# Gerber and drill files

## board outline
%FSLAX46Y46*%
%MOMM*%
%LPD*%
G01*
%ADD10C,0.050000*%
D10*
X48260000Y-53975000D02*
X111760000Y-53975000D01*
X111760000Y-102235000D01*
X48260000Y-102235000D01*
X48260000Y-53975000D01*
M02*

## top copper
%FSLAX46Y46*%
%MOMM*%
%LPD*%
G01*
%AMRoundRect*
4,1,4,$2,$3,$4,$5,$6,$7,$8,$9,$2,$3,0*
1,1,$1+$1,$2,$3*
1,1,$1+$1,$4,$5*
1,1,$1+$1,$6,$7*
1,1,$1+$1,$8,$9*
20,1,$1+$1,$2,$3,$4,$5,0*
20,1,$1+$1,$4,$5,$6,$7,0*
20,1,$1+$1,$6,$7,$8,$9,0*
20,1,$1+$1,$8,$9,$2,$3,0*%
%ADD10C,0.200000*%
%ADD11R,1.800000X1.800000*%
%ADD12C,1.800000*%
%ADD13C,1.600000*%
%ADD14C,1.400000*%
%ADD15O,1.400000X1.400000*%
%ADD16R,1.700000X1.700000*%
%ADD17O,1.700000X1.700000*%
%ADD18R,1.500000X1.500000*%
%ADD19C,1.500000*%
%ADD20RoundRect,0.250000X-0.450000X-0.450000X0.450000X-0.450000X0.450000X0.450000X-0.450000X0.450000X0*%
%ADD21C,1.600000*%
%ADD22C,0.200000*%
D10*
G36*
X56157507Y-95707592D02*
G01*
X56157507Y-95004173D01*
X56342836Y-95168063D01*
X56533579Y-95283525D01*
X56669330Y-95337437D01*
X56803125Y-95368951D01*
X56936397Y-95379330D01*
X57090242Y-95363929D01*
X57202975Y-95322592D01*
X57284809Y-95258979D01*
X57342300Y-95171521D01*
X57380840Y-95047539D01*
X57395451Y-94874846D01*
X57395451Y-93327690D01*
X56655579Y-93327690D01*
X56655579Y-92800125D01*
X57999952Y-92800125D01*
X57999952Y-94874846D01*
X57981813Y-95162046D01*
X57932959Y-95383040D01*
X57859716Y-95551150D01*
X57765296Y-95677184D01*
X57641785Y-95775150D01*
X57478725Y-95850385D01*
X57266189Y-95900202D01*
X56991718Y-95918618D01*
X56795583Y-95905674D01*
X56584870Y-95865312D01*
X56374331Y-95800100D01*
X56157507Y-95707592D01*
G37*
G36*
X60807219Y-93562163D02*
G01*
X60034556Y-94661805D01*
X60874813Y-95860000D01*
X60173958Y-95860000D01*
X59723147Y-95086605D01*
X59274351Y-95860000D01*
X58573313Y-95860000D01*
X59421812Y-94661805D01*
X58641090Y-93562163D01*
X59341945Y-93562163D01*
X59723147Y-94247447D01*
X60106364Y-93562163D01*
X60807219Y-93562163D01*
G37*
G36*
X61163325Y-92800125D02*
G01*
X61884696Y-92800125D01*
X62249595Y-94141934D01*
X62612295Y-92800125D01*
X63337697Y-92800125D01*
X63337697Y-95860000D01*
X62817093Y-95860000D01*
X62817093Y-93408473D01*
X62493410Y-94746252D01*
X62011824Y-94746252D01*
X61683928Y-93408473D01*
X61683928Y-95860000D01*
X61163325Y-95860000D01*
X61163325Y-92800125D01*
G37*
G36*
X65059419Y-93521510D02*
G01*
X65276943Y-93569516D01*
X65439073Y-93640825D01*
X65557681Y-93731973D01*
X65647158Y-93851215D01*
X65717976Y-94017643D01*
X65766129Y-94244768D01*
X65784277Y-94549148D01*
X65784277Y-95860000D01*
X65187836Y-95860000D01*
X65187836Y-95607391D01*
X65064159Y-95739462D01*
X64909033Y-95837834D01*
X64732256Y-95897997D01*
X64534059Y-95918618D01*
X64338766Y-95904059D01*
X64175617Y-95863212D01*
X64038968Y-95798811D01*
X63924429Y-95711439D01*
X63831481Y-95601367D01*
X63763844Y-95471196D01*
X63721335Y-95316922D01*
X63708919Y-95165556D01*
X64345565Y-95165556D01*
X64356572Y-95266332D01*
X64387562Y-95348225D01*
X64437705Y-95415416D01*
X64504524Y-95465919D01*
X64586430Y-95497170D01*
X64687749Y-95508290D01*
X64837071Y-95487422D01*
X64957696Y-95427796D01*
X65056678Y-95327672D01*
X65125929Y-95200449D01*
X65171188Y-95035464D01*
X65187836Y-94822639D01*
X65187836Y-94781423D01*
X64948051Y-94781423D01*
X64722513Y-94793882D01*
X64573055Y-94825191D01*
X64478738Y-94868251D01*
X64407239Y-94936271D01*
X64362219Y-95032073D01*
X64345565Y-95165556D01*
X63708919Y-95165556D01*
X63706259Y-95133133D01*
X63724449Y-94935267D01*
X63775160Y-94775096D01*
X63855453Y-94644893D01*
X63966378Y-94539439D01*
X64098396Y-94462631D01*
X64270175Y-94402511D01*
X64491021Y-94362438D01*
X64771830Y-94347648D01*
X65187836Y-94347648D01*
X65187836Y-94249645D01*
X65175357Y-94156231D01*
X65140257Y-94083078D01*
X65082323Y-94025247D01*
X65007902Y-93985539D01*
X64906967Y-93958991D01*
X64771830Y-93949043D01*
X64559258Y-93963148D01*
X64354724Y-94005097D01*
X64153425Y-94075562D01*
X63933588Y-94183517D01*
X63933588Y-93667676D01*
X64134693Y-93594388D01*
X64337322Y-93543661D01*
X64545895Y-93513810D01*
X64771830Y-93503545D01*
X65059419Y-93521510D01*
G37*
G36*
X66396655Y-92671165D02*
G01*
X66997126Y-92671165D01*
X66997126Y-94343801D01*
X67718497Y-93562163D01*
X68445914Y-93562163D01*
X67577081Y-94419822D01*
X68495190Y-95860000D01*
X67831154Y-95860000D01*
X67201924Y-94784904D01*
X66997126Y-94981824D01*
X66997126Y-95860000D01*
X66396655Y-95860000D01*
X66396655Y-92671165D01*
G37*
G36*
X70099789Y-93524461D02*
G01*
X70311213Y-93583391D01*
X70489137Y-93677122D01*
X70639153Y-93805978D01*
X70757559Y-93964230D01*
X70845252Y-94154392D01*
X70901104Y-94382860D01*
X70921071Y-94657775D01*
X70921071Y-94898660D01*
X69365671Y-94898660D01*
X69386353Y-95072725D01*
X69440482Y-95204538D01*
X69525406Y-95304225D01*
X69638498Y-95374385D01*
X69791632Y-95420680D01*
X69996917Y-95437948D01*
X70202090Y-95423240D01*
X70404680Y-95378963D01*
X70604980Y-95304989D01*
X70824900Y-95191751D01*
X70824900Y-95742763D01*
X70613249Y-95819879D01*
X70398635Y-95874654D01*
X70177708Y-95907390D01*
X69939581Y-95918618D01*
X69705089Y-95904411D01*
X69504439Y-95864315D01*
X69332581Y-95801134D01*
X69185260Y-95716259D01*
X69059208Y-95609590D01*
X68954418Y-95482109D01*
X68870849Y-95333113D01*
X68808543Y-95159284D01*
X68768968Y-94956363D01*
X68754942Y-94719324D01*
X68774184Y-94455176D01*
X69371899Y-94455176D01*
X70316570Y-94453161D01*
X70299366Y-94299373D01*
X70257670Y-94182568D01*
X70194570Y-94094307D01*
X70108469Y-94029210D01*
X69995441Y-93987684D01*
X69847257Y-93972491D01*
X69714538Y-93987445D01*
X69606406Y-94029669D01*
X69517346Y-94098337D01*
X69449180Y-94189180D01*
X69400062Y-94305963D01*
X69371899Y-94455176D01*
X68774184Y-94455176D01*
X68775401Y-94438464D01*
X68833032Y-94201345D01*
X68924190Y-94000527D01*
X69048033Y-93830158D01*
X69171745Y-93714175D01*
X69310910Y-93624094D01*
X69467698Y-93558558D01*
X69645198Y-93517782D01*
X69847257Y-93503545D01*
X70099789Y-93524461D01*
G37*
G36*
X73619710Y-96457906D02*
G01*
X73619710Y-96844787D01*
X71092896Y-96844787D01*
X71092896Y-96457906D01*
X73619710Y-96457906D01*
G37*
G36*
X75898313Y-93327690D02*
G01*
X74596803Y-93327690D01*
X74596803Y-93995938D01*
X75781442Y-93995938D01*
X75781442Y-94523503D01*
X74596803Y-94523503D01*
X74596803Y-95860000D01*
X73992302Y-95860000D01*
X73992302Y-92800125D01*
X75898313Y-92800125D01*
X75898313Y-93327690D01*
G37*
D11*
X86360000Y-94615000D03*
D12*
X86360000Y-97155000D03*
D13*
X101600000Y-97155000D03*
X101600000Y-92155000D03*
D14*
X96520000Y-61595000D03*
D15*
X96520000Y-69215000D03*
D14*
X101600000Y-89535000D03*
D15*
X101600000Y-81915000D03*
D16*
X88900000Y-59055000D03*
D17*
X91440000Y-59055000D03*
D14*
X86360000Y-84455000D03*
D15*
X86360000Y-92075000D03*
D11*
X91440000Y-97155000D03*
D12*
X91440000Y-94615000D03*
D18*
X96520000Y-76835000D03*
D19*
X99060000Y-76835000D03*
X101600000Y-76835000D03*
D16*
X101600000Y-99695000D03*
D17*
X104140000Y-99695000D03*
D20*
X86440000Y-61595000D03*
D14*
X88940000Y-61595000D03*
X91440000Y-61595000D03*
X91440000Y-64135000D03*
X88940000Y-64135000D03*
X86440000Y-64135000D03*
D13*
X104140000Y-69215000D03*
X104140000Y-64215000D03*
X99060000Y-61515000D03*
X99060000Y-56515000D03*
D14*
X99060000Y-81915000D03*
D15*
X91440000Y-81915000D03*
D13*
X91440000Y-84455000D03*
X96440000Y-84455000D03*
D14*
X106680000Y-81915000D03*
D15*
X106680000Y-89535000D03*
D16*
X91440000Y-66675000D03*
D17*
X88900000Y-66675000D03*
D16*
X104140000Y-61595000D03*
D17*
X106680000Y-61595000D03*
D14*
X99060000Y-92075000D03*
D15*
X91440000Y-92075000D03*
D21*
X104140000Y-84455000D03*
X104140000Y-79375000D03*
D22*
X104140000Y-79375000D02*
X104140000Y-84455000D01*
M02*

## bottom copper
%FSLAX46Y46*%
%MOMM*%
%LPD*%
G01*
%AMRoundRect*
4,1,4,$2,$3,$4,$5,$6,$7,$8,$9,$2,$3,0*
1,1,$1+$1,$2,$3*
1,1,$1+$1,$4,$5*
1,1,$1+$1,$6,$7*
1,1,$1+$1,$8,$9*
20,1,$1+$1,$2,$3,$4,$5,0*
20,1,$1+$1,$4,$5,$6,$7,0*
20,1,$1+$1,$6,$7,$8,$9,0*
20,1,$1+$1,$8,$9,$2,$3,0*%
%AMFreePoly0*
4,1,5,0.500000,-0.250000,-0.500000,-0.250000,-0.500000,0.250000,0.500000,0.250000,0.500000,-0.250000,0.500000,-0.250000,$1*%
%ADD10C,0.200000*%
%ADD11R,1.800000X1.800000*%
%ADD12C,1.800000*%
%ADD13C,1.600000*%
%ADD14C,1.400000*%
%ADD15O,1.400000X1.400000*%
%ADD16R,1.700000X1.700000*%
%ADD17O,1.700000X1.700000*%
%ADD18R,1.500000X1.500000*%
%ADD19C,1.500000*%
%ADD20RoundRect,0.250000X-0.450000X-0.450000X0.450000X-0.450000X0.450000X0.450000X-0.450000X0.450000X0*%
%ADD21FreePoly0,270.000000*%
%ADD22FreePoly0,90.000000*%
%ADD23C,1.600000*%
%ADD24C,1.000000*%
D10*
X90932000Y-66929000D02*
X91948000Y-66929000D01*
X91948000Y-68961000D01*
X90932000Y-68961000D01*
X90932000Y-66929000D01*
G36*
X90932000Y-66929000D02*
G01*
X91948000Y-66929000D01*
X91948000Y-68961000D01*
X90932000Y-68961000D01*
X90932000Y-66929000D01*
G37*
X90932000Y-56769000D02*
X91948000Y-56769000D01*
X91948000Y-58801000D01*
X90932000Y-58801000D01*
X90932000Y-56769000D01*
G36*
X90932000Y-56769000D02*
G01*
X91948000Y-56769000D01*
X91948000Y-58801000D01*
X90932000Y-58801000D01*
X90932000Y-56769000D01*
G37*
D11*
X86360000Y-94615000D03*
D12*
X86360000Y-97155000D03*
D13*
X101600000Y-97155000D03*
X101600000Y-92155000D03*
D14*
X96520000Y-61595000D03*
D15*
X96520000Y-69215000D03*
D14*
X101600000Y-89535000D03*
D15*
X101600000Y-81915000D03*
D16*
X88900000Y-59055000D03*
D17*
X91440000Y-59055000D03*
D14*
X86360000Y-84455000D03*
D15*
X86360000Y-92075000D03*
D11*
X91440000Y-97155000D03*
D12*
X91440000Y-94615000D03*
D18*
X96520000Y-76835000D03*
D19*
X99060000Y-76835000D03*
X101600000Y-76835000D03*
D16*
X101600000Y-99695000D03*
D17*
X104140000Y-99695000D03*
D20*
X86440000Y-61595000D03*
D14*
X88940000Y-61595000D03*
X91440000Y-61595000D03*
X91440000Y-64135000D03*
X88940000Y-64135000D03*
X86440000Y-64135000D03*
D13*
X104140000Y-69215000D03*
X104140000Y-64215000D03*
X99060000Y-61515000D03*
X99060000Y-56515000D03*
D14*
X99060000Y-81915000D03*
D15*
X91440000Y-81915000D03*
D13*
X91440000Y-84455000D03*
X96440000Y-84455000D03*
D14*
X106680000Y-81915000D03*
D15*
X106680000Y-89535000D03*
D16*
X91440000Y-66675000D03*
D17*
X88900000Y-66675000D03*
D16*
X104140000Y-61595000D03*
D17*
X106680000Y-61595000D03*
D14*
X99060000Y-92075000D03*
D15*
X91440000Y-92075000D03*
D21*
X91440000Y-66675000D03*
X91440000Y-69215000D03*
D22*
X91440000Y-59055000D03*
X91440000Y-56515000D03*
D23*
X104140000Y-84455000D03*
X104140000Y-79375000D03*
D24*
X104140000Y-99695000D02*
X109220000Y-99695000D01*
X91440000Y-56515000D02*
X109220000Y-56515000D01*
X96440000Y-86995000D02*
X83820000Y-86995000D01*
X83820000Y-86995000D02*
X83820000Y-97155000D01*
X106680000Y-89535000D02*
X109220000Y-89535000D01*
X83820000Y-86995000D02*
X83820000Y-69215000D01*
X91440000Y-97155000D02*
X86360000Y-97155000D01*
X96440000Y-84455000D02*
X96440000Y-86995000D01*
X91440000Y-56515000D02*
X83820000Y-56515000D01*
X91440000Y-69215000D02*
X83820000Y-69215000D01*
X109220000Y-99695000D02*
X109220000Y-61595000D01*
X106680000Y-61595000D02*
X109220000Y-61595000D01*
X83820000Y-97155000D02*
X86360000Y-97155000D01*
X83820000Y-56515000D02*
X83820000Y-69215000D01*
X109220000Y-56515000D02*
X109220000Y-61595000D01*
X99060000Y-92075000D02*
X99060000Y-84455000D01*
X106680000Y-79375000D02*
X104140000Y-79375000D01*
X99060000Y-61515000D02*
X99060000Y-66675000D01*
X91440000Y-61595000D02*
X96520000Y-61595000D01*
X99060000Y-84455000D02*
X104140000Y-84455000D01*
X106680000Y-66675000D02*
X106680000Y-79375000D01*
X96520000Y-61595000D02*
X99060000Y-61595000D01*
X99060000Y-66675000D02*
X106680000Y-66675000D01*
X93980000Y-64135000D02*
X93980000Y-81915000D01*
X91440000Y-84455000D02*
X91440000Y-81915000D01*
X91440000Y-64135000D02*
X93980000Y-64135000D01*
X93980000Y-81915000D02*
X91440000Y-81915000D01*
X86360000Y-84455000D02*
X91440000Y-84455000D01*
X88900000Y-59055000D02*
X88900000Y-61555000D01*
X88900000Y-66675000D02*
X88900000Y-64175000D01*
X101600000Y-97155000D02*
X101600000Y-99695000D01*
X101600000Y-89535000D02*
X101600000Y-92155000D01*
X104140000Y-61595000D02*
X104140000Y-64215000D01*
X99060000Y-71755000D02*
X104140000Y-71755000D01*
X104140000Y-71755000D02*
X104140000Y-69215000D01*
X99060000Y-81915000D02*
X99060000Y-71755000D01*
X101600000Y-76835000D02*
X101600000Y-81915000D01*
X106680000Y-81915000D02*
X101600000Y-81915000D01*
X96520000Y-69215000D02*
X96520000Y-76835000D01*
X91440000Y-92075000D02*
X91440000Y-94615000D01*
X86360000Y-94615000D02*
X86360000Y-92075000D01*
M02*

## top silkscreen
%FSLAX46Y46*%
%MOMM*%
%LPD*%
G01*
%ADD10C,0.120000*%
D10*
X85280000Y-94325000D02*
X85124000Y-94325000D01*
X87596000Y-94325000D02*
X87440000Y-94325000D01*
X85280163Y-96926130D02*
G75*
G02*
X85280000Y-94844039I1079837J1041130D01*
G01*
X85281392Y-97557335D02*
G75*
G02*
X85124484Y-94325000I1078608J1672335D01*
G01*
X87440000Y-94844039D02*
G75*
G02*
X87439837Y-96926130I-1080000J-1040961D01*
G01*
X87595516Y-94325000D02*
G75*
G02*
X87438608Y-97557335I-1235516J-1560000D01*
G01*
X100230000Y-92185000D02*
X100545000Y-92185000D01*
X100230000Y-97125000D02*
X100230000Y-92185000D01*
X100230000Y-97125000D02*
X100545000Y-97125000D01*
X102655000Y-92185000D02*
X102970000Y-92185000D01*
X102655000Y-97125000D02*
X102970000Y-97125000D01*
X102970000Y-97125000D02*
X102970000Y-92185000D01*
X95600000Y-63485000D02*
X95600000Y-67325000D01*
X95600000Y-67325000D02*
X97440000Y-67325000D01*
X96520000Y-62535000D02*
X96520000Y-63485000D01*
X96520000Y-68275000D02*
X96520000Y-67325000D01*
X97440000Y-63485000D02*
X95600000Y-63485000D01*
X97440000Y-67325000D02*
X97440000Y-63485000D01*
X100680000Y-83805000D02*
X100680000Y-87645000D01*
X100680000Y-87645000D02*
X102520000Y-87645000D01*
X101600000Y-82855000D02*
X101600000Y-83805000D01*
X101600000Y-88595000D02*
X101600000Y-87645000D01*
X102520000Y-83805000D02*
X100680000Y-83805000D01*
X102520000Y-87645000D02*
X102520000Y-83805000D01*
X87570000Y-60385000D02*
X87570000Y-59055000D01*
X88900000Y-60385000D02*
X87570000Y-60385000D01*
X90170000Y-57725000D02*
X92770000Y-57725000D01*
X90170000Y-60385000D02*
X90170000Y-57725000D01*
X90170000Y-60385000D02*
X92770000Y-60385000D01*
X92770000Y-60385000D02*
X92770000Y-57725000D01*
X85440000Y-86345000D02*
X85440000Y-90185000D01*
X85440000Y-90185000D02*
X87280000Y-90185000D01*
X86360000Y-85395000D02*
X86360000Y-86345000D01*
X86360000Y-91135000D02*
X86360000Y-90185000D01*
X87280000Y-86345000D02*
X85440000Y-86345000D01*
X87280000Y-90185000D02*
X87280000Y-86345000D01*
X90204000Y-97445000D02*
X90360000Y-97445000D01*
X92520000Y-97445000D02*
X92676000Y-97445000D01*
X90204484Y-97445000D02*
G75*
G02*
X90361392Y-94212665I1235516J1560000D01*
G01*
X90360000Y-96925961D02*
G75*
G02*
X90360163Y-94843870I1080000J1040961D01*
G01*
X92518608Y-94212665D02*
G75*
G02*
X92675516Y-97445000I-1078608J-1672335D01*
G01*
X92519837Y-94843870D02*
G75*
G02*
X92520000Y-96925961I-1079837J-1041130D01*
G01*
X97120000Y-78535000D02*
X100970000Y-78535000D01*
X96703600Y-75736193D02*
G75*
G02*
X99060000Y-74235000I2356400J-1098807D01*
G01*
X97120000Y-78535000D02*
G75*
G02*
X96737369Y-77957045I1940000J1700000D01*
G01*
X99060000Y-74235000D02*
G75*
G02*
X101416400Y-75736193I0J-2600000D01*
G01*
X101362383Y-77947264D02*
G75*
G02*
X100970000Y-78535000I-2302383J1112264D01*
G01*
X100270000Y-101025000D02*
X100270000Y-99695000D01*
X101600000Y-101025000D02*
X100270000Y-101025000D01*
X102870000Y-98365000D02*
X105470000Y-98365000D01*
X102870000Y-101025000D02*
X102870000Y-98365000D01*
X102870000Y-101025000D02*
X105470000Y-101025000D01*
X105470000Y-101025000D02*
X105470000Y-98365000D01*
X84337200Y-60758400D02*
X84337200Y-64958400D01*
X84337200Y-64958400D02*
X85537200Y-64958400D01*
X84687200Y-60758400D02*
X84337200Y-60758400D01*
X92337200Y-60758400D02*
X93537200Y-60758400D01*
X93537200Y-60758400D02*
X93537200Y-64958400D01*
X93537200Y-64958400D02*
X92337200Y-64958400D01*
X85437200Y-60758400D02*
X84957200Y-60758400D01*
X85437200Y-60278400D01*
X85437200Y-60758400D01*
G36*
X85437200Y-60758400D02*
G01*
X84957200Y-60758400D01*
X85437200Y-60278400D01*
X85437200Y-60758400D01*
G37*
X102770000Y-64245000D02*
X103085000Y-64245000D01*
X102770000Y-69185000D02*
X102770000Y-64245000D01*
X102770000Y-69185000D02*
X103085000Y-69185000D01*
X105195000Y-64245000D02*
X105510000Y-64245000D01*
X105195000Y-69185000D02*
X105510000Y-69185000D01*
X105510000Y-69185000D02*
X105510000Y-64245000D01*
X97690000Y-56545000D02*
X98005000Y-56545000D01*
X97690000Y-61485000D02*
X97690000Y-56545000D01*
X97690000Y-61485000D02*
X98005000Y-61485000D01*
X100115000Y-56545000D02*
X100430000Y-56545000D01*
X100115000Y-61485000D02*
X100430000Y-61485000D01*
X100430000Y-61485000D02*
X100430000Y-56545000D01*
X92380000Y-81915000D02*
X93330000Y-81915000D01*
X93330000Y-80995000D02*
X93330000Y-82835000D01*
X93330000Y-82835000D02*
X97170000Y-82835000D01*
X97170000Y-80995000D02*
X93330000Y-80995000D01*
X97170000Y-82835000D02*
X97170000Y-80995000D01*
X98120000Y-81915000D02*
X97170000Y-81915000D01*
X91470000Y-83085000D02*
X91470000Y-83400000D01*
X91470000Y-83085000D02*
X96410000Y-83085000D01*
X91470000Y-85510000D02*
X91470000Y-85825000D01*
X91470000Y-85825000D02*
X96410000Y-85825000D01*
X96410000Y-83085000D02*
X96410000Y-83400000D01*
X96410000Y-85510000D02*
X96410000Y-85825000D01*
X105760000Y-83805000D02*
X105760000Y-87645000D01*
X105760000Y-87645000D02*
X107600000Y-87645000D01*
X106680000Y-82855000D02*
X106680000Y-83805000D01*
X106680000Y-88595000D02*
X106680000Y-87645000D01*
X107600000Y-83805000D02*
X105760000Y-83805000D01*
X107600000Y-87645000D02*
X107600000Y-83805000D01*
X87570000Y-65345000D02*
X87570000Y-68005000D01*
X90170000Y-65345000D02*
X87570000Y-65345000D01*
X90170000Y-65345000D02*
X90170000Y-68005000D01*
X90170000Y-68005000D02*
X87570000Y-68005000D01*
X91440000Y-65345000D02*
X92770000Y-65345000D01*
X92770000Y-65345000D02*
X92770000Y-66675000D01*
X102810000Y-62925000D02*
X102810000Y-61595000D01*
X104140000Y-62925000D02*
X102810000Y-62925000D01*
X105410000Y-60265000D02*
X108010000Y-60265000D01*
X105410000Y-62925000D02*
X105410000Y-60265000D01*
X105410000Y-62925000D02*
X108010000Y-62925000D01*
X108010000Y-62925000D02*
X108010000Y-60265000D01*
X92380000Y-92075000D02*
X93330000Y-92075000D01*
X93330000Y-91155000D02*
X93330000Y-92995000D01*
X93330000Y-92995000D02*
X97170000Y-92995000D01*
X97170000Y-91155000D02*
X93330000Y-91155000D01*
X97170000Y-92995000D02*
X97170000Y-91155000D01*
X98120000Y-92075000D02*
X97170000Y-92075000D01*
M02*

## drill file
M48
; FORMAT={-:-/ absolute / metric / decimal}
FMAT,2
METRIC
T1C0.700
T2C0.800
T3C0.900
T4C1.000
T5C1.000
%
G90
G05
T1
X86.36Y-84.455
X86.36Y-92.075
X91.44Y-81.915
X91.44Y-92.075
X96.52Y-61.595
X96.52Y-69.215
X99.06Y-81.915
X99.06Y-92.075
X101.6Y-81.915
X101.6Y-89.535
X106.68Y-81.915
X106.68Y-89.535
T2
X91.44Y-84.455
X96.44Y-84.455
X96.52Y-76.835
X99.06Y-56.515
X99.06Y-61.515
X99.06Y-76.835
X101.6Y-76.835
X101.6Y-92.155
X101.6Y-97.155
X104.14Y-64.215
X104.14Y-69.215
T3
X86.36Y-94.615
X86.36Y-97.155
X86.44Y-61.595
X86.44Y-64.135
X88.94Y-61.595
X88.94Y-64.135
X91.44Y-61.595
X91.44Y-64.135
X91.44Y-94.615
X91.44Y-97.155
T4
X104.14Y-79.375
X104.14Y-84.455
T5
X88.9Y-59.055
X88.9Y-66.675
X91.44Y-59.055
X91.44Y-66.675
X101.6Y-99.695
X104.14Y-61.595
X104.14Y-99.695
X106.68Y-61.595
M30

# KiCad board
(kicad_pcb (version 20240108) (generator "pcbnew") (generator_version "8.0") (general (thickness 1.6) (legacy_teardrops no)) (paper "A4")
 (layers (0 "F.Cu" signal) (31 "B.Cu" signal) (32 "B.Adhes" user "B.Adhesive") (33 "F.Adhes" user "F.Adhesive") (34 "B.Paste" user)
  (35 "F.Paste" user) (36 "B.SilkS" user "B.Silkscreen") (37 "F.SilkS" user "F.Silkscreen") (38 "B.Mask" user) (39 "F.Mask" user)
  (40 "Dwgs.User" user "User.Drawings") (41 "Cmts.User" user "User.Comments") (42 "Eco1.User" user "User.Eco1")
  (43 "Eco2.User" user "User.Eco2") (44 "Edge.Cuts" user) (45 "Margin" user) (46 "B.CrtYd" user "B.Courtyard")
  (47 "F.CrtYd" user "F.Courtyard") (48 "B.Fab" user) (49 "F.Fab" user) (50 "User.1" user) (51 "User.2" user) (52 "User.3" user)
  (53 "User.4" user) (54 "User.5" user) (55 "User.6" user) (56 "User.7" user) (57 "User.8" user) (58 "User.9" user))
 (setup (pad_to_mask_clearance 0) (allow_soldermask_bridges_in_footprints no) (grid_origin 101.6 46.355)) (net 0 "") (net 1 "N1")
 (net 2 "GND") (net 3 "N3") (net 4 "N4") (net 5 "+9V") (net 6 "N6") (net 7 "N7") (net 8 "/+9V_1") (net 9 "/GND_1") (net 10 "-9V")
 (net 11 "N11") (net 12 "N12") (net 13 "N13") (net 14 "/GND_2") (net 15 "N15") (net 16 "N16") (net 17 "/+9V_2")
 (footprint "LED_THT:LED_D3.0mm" (layer "F.Cu") (at 86.36 94.615 -90)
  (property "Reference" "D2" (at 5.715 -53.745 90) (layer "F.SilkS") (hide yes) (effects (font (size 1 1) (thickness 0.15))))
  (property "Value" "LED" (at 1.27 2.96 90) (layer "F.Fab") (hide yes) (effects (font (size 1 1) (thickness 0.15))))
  (fp_line (start -0.29 1.08) (end -0.29 1.236) (stroke (width 0.12) (type solid)) (layer "F.SilkS"))
  (fp_line (start -0.29 -1.236) (end -0.29 -1.08) (stroke (width 0.12) (type solid)) (layer "F.SilkS"))
  (fp_arc (start 2.31113 1.079837) (mid 1.270117 1.5) (end 0.229039 1.08) (stroke (width 0.12) (type solid)) (layer "F.SilkS"))
  (fp_arc (start 2.942335 1.078608) (mid 1.366487 1.987659) (end -0.29 1.235516) (stroke (width 0.12) (type solid)) (layer "F.SilkS"))
  (fp_arc (start 0.229039 -1.08) (mid 1.270117 -1.5) (end 2.31113 -1.079837) (stroke (width 0.12) (type solid)) (layer "F.SilkS"))
  (fp_arc (start -0.29 -1.235516) (mid 1.366487 -1.987659) (end 2.942335 -1.078608) (stroke (width 0.12) (type solid)) (layer "F.SilkS"))
  (pad "1" thru_hole rect (at 0 0 270) (size 1.8 1.8) (drill 0.9) (layers "*.Cu" "*.Mask") (remove_unused_layers no) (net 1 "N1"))
  (pad "2" thru_hole circle (at 2.54 0 270) (size 1.8 1.8) (drill 0.9) (layers "*.Cu" "*.Mask") (remove_unused_layers no) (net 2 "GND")))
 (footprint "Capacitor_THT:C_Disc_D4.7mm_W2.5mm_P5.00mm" (layer "F.Cu") (at 101.6 97.155 90)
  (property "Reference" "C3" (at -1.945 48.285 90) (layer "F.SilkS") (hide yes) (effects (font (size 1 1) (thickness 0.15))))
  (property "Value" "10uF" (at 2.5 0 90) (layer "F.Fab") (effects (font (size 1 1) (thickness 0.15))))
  (fp_line (start 4.97 -1.37) (end 4.97 -1.055) (stroke (width 0.12) (type solid)) (layer "F.SilkS"))
  (fp_line (start 0.03 -1.37) (end 4.97 -1.37) (stroke (width 0.12) (type solid)) (layer "F.SilkS"))
  (fp_line (start 0.03 -1.37) (end 0.03 -1.055) (stroke (width 0.12) (type solid)) (layer "F.SilkS"))
  (fp_line (start 4.97 1.055) (end 4.97 1.37) (stroke (width 0.12) (type solid)) (layer "F.SilkS"))
  (fp_line (start 0.03 1.055) (end 0.03 1.37) (stroke (width 0.12) (type solid)) (layer "F.SilkS"))
  (fp_line (start 0.03 1.37) (end 4.97 1.37) (stroke (width 0.12) (type solid)) (layer "F.SilkS"))
  (pad "1" thru_hole circle (at 0 0 90) (size 1.6 1.6) (drill 0.8) (layers "*.Cu" "*.Mask") (remove_unused_layers no) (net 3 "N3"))
  (pad "2" thru_hole circle (at 5 0 90) (size 1.6 1.6) (drill 0.8) (layers "*.Cu" "*.Mask") (remove_unused_layers no) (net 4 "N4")))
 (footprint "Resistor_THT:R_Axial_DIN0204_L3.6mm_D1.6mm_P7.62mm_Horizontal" (layer "F.Cu") (at 96.52 61.595 -90)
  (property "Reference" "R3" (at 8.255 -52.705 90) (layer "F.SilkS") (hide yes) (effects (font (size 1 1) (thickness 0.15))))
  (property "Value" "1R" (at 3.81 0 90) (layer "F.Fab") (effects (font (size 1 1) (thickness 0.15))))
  (fp_line (start 1.89 0.92) (end 5.73 0.92) (stroke (width 0.12) (type solid)) (layer "F.SilkS"))
  (fp_line (start 5.73 0.92) (end 5.73 -0.92) (stroke (width 0.12) (type solid)) (layer "F.SilkS"))
  (fp_line (start 0.94 0) (end 1.89 0) (stroke (width 0.12) (type solid)) (layer "F.SilkS"))
  (fp_line (start 6.68 0) (end 5.73 0) (stroke (width 0.12) (type solid)) (layer "F.SilkS"))
  (fp_line (start 1.89 -0.92) (end 1.89 0.92) (stroke (width 0.12) (type solid)) (layer "F.SilkS"))
  (fp_line (start 5.73 -0.92) (end 1.89 -0.92) (stroke (width 0.12) (type solid)) (layer "F.SilkS"))
  (pad "1" thru_hole circle (at 0 0 270) (size 1.4 1.4) (drill 0.7) (layers "*.Cu" "*.Mask") (remove_unused_layers no) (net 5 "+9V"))
  (pad "2" thru_hole oval (at 7.62 0 270) (size 1.4 1.4) (drill 0.7) (layers "*.Cu" "*.Mask") (remove_unused_layers no) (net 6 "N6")))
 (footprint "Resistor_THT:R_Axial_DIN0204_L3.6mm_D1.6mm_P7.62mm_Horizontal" (layer "F.Cu") (at 101.6 89.535 90)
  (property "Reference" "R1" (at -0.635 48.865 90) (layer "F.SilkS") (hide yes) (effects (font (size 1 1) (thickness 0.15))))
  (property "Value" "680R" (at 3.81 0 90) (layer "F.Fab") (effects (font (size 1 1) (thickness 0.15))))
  (fp_line (start 5.73 -0.92) (end 1.89 -0.92) (stroke (width 0.12) (type solid)) (layer "F.SilkS"))
  (fp_line (start 1.89 -0.92) (end 1.89 0.92) (stroke (width 0.12) (type solid)) (layer "F.SilkS"))
  (fp_line (start 6.68 0) (end 5.73 0) (stroke (width 0.12) (type solid)) (layer "F.SilkS"))
  (fp_line (start 0.94 0) (end 1.89 0) (stroke (width 0.12) (type solid)) (layer "F.SilkS"))
  (fp_line (start 5.73 0.92) (end 5.73 -0.92) (stroke (width 0.12) (type solid)) (layer "F.SilkS"))
  (fp_line (start 1.89 0.92) (end 5.73 0.92) (stroke (width 0.12) (type solid)) (layer "F.SilkS"))
  (pad "1" thru_hole circle (at 0 0 90) (size 1.4 1.4) (drill 0.7) (layers "*.Cu" "*.Mask") (remove_unused_layers no) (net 4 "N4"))
  (pad "2" thru_hole oval (at 7.62 0 90) (size 1.4 1.4) (drill 0.7) (layers "*.Cu" "*.Mask") (remove_unused_layers no) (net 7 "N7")))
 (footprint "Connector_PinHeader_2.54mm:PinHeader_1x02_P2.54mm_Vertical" (layer "F.Cu") (at 88.9 59.055 90)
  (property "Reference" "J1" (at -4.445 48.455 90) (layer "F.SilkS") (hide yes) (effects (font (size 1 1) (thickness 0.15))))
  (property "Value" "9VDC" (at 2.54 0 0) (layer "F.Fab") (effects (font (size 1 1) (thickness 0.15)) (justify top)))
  (fp_line (start -1.33 -1.33) (end 0 -1.33) (stroke (width 0.12) (type solid)) (layer "F.SilkS"))
  (fp_line (start -1.33 0) (end -1.33 -1.33) (stroke (width 0.12) (type solid)) (layer "F.SilkS"))
  (fp_line (start 1.33 1.27) (end 1.33 3.87) (stroke (width 0.12) (type solid)) (layer "F.SilkS"))
  (fp_line (start -1.33 1.27) (end 1.33 1.27) (stroke (width 0.12) (type solid)) (layer "F.SilkS"))
  (fp_line (start -1.33 1.27) (end -1.33 3.87) (stroke (width 0.12) (type solid)) (layer "F.SilkS"))
  (fp_line (start -1.33 3.87) (end 1.33 3.87) (stroke (width 0.12) (type solid)) (layer "F.SilkS"))
  (pad "1" thru_hole rect (at 0 0 90) (size 1.7 1.7) (drill 1) (layers "*.Cu" "*.Mask") (remove_unused_layers no) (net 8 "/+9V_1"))
  (pad "2" thru_hole oval (at 0 2.54 90) (size 1.7 1.7) (drill 1) (layers "*.Cu" "*.Mask") (remove_unused_layers no) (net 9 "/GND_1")))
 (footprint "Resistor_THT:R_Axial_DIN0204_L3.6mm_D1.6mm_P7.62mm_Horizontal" (layer "F.Cu") (at 86.36 84.455 -90)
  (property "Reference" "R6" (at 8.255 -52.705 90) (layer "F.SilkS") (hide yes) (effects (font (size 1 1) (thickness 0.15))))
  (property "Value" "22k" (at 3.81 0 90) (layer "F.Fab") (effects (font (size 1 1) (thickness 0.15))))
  (fp_line (start 1.89 0.92) (end 5.73 0.92) (stroke (width 0.12) (type solid)) (layer "F.SilkS"))
  (fp_line (start 5.73 0.92) (end 5.73 -0.92) (stroke (width 0.12) (type solid)) (layer "F.SilkS"))
  (fp_line (start 0.94 0) (end 1.89 0) (stroke (width 0.12) (type solid)) (layer "F.SilkS"))
  (fp_line (start 6.68 0) (end 5.73 0) (stroke (width 0.12) (type solid)) (layer "F.SilkS"))
  (fp_line (start 1.89 -0.92) (end 1.89 0.92) (stroke (width 0.12) (type solid)) (layer "F.SilkS"))
  (fp_line (start 5.73 -0.92) (end 1.89 -0.92) (stroke (width 0.12) (type solid)) (layer "F.SilkS"))
  (pad "1" thru_hole circle (at 0 0 270) (size 1.4 1.4) (drill 0.7) (layers "*.Cu" "*.Mask") (remove_unused_layers no) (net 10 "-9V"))
  (pad "2" thru_hole oval (at 7.62 0 270) (size 1.4 1.4) (drill 0.7) (layers "*.Cu" "*.Mask") (remove_unused_layers no) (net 1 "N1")))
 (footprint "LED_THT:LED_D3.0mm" (layer "F.Cu") (at 91.44 97.155 90)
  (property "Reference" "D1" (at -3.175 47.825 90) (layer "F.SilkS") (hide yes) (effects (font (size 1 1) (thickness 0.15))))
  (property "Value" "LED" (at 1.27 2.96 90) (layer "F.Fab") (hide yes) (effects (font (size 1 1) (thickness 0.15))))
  (fp_line (start -0.29 -1.236) (end -0.29 -1.08) (stroke (width 0.12) (type solid)) (layer "F.SilkS"))
  (fp_line (start -0.29 1.08) (end -0.29 1.236) (stroke (width 0.12) (type solid)) (layer "F.SilkS"))
  (fp_arc (start -0.29 -1.235516) (mid 1.366487 -1.987659) (end 2.942335 -1.078608) (stroke (width 0.12) (type solid)) (layer "F.SilkS"))
  (fp_arc (start 0.229039 -1.08) (mid 1.270117 -1.5) (end 2.31113 -1.079837) (stroke (width 0.12) (type solid)) (layer "F.SilkS"))
  (fp_arc (start 2.942335 1.078608) (mid 1.366487 1.987659) (end -0.29 1.235516) (stroke (width 0.12) (type solid)) (layer "F.SilkS"))
  (fp_arc (start 2.31113 1.079837) (mid 1.270117 1.5) (end 0.229039 1.08) (stroke (width 0.12) (type solid)) (layer "F.SilkS"))
  (pad "1" thru_hole rect (at 0 0 90) (size 1.8 1.8) (drill 0.9) (layers "*.Cu" "*.Mask") (remove_unused_layers no) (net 2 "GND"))
  (pad "2" thru_hole circle (at 2.54 0 90) (size 1.8 1.8) (drill 0.9) (layers "*.Cu" "*.Mask") (remove_unused_layers no) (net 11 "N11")))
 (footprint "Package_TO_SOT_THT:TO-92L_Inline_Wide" (layer "F.Cu") (at 96.52 76.835)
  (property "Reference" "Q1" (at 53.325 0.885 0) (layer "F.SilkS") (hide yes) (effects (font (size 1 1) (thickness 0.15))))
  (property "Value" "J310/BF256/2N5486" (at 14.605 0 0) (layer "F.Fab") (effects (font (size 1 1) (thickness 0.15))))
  (fp_line (start 0.6 1.7) (end 4.45 1.7) (stroke (width 0.12) (type solid)) (layer "F.SilkS"))
  (fp_arc (start 0.1836 -1.098807) (mid 1.143021 -2.192817) (end 2.54 -2.6) (stroke (width 0.12) (type solid)) (layer "F.SilkS"))
  (fp_arc (start 0.6 1.7) (mid 0.389183 1.423933) (end 0.217369 1.122045) (stroke (width 0.12) (type solid)) (layer "F.SilkS"))
  (fp_arc (start 2.54 -2.6) (mid 3.936979 -2.192818) (end 4.8964 -1.098807) (stroke (width 0.12) (type solid)) (layer "F.SilkS"))
  (fp_arc (start 4.842383 1.112264) (mid 4.666594 1.419753) (end 4.45 1.7) (stroke (width 0.12) (type solid)) (layer "F.SilkS"))
  (pad "1" thru_hole rect (at 0 0) (size 1.5 1.5) (drill 0.8) (layers "*.Cu" "*.Mask") (remove_unused_layers no) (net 6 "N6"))
  (pad "2" thru_hole circle (at 2.54 0) (size 1.5 1.5) (drill 0.8) (layers "*.Cu" "*.Mask") (remove_unused_layers no) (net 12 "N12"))
  (pad "3" thru_hole circle (at 5.08 0) (size 1.5 1.5) (drill 0.8) (layers "*.Cu" "*.Mask") (remove_unused_layers no) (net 7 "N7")))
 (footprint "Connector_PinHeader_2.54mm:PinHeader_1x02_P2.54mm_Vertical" (layer "F.Cu") (at 101.6 99.695 90)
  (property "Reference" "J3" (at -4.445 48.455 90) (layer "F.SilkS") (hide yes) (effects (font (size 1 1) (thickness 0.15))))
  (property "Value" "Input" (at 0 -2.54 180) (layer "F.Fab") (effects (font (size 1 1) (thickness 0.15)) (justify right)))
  (fp_line (start -1.33 -1.33) (end 0 -1.33) (stroke (width 0.12) (type solid)) (layer "F.SilkS"))
  (fp_line (start -1.33 0) (end -1.33 -1.33) (stroke (width 0.12) (type solid)) (layer "F.SilkS"))
  (fp_line (start 1.33 1.27) (end 1.33 3.87) (stroke (width 0.12) (type solid)) (layer "F.SilkS"))
  (fp_line (start -1.33 1.27) (end 1.33 1.27) (stroke (width 0.12) (type solid)) (layer "F.SilkS"))
  (fp_line (start -1.33 1.27) (end -1.33 3.87) (stroke (width 0.12) (type solid)) (layer "F.SilkS"))
  (fp_line (start -1.33 3.87) (end 1.33 3.87) (stroke (width 0.12) (type solid)) (layer "F.SilkS"))
  (pad "1" thru_hole rect (at 0 0 90) (size 1.7 1.7) (drill 1) (layers "*.Cu" "*.Mask") (remove_unused_layers no) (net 3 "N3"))
  (pad "2" thru_hole oval (at 0 2.54 90) (size 1.7 1.7) (drill 1) (layers "*.Cu" "*.Mask") (remove_unused_layers no) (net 2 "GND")))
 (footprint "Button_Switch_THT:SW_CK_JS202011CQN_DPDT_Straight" (layer "F.Cu") (at 86.44 61.595)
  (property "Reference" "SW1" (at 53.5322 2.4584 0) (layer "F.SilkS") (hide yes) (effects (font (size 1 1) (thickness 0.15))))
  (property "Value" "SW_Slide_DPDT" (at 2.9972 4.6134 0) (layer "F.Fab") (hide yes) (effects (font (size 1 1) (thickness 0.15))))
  (fp_line (start -2.1028 -0.8366) (end -2.1028 3.3634) (stroke (width 0.12) (type solid)) (layer "F.SilkS"))
  (fp_line (start -2.1028 3.3634) (end -0.9028 3.3634) (stroke (width 0.12) (type solid)) (layer "F.SilkS"))
  (fp_line (start -1.7528 -0.8366) (end -2.1028 -0.8366) (stroke (width 0.12) (type solid)) (layer "F.SilkS"))
  (fp_line (start 5.8972 -0.8366) (end 7.0972 -0.8366) (stroke (width 0.12) (type solid)) (layer "F.SilkS"))
  (fp_line (start 7.0972 -0.8366) (end 7.0972 3.3634) (stroke (width 0.12) (type solid)) (layer "F.SilkS"))
  (fp_line (start 7.0972 3.3634) (end 5.8972 3.3634) (stroke (width 0.12) (type solid)) (layer "F.SilkS"))
  (fp_poly
   (pts (xy -1.0028 -0.8366) (xy -1.4828 -0.8366) (xy -1.0028 -1.3166) (xy -1.0028 -0.8366)) (stroke (width 0.12) (type solid)) (fill solid)
   (layer "F.SilkS"))
  (pad "1" thru_hole roundrect (at 0 0) (size 1.4 1.4) (drill 0.9) (layers "*.Cu" "*.Mask") (remove_unused_layers no)
   (roundrect_rratio 0.1785714286) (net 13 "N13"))
  (pad "2" thru_hole circle (at 2.5 0) (size 1.4 1.4) (drill 0.9) (layers "*.Cu" "*.Mask") (remove_unused_layers no) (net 8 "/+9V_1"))
  (pad "3" thru_hole circle (at 5 0) (size 1.4 1.4) (drill 0.9) (layers "*.Cu" "*.Mask") (remove_unused_layers no) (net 5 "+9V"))
  (pad "4" thru_hole circle (at 5 2.54) (size 1.4 1.4) (drill 0.9) (layers "*.Cu" "*.Mask") (remove_unused_layers no) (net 10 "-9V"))
  (pad "5" thru_hole circle (at 2.5 2.54) (size 1.4 1.4) (drill 0.9) (layers "*.Cu" "*.Mask") (remove_unused_layers no) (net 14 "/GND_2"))
  (pad "6" thru_hole circle (at 0 2.54) (size 1.4 1.4) (drill 0.9) (layers "*.Cu" "*.Mask") (remove_unused_layers no) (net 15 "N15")))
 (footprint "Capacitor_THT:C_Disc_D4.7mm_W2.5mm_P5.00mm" (layer "F.Cu") (at 104.14 69.215 90)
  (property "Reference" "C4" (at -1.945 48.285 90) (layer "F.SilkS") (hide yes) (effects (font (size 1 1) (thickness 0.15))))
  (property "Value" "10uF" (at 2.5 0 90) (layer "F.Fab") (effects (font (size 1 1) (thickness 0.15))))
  (fp_line (start 4.97 -1.37) (end 4.97 -1.055) (stroke (width 0.12) (type solid)) (layer "F.SilkS"))
  (fp_line (start 0.03 -1.37) (end 4.97 -1.37) (stroke (width 0.12) (type solid)) (layer "F.SilkS"))
  (fp_line (start 0.03 -1.37) (end 0.03 -1.055) (stroke (width 0.12) (type solid)) (layer "F.SilkS"))
  (fp_line (start 4.97 1.055) (end 4.97 1.37) (stroke (width 0.12) (type solid)) (layer "F.SilkS"))
  (fp_line (start 0.03 1.055) (end 0.03 1.37) (stroke (width 0.12) (type solid)) (layer "F.SilkS"))
  (fp_line (start 0.03 1.37) (end 4.97 1.37) (stroke (width 0.12) (type solid)) (layer "F.SilkS"))
  (pad "1" thru_hole circle (at 0 0 90) (size 1.6 1.6) (drill 0.8) (layers "*.Cu" "*.Mask") (remove_unused_layers no) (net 12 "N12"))
  (pad "2" thru_hole circle (at 5 0 90) (size 1.6 1.6) (drill 0.8) (layers "*.Cu" "*.Mask") (remove_unused_layers no) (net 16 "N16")))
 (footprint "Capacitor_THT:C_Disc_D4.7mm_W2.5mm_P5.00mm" (layer "F.Cu") (at 99.06 61.515 90)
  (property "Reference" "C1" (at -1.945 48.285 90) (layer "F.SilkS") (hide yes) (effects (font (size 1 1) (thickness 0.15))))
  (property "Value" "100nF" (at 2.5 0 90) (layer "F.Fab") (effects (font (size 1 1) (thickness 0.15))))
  (fp_line (start 4.97 -1.37) (end 4.97 -1.055) (stroke (width 0.12) (type solid)) (layer "F.SilkS"))
  (fp_line (start 0.03 -1.37) (end 4.97 -1.37) (stroke (width 0.12) (type solid)) (layer "F.SilkS"))
  (fp_line (start 0.03 -1.37) (end 0.03 -1.055) (stroke (width 0.12) (type solid)) (layer "F.SilkS"))
  (fp_line (start 4.97 1.055) (end 4.97 1.37) (stroke (width 0.12) (type solid)) (layer "F.SilkS"))
  (fp_line (start 0.03 1.055) (end 0.03 1.37) (stroke (width 0.12) (type solid)) (layer "F.SilkS"))
  (fp_line (start 0.03 1.37) (end 4.97 1.37) (stroke (width 0.12) (type solid)) (layer "F.SilkS"))
  (pad "1" thru_hole circle (at 0 0 90) (size 1.6 1.6) (drill 0.8) (layers "*.Cu" "*.Mask") (remove_unused_layers no) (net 5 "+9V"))
  (pad "2" thru_hole circle (at 5 0 90) (size 1.6 1.6) (drill 0.8) (layers "*.Cu" "*.Mask") (remove_unused_layers no) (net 2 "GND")))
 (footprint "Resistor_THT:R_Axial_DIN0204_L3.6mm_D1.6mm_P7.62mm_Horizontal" (layer "F.Cu") (at 99.06 81.915 180)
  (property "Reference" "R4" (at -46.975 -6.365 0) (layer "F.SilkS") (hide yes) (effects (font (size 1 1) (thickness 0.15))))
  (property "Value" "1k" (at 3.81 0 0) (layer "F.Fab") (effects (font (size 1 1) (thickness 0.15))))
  (fp_line (start 6.68 0) (end 5.73 0) (stroke (width 0.12) (type solid)) (layer "F.SilkS"))
  (fp_line (start 5.73 0.92) (end 5.73 -0.92) (stroke (width 0.12) (type solid)) (layer "F.SilkS"))
  (fp_line (start 5.73 -0.92) (end 1.89 -0.92) (stroke (width 0.12) (type solid)) (layer "F.SilkS"))
  (fp_line (start 1.89 0.92) (end 5.73 0.92) (stroke (width 0.12) (type solid)) (layer "F.SilkS"))
  (fp_line (start 1.89 -0.92) (end 1.89 0.92) (stroke (width 0.12) (type solid)) (layer "F.SilkS"))
  (fp_line (start 0.94 0) (end 1.89 0) (stroke (width 0.12) (type solid)) (layer "F.SilkS"))
  (pad "1" thru_hole circle (at 0 0 180) (size 1.4 1.4) (drill 0.7) (layers "*.Cu" "*.Mask") (remove_unused_layers no) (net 12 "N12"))
  (pad "2" thru_hole oval (at 7.62 0 180) (size 1.4 1.4) (drill 0.7) (layers "*.Cu" "*.Mask") (remove_unused_layers no) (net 10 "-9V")))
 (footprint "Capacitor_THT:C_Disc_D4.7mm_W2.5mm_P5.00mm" (layer "F.Cu") (at 91.44 84.455)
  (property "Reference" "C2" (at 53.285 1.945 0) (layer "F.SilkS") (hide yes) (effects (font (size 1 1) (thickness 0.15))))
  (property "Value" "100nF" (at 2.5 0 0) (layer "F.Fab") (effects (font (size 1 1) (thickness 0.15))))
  (fp_line (start 0.03 -1.37) (end 0.03 -1.055) (stroke (width 0.12) (type solid)) (layer "F.SilkS"))
  (fp_line (start 0.03 -1.37) (end 4.97 -1.37) (stroke (width 0.12) (type solid)) (layer "F.SilkS"))
  (fp_line (start 0.03 1.055) (end 0.03 1.37) (stroke (width 0.12) (type solid)) (layer "F.SilkS"))
  (fp_line (start 0.03 1.37) (end 4.97 1.37) (stroke (width 0.12) (type solid)) (layer "F.SilkS"))
  (fp_line (start 4.97 -1.37) (end 4.97 -1.055) (stroke (width 0.12) (type solid)) (layer "F.SilkS"))
  (fp_line (start 4.97 1.055) (end 4.97 1.37) (stroke (width 0.12) (type solid)) (layer "F.SilkS"))
  (pad "1" thru_hole circle (at 0 0) (size 1.6 1.6) (drill 0.8) (layers "*.Cu" "*.Mask") (remove_unused_layers no) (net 10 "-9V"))
  (pad "2" thru_hole circle (at 5 0) (size 1.6 1.6) (drill 0.8) (layers "*.Cu" "*.Mask") (remove_unused_layers no) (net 2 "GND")))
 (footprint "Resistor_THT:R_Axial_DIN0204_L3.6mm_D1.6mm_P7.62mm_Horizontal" (layer "F.Cu") (at 106.68 81.915 -90)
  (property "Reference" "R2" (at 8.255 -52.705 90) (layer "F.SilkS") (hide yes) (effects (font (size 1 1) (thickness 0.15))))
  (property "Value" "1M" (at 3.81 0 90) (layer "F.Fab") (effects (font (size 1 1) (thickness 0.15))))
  (fp_line (start 1.89 0.92) (end 5.73 0.92) (stroke (width 0.12) (type solid)) (layer "F.SilkS"))
  (fp_line (start 5.73 0.92) (end 5.73 -0.92) (stroke (width 0.12) (type solid)) (layer "F.SilkS"))
  (fp_line (start 0.94 0) (end 1.89 0) (stroke (width 0.12) (type solid)) (layer "F.SilkS"))
  (fp_line (start 6.68 0) (end 5.73 0) (stroke (width 0.12) (type solid)) (layer "F.SilkS"))
  (fp_line (start 1.89 -0.92) (end 1.89 0.92) (stroke (width 0.12) (type solid)) (layer "F.SilkS"))
  (fp_line (start 5.73 -0.92) (end 1.89 -0.92) (stroke (width 0.12) (type solid)) (layer "F.SilkS"))
  (pad "1" thru_hole circle (at 0 0 270) (size 1.4 1.4) (drill 0.7) (layers "*.Cu" "*.Mask") (remove_unused_layers no) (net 7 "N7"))
  (pad "2" thru_hole oval (at 7.62 0 270) (size 1.4 1.4) (drill 0.7) (layers "*.Cu" "*.Mask") (remove_unused_layers no) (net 2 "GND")))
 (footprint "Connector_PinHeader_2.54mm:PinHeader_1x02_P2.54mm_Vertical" (layer "F.Cu") (at 91.44 66.675 -90)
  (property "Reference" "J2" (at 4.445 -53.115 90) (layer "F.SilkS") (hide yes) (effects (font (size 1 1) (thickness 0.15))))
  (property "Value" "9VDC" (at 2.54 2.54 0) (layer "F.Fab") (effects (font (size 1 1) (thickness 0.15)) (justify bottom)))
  (fp_line (start -1.33 3.87) (end 1.33 3.87) (stroke (width 0.12) (type solid)) (layer "F.SilkS"))
  (fp_line (start -1.33 1.27) (end -1.33 3.87) (stroke (width 0.12) (type solid)) (layer "F.SilkS"))
  (fp_line (start -1.33 1.27) (end 1.33 1.27) (stroke (width 0.12) (type solid)) (layer "F.SilkS"))
  (fp_line (start 1.33 1.27) (end 1.33 3.87) (stroke (width 0.12) (type solid)) (layer "F.SilkS"))
  (fp_line (start -1.33 0) (end -1.33 -1.33) (stroke (width 0.12) (type solid)) (layer "F.SilkS"))
  (fp_line (start -1.33 -1.33) (end 0 -1.33) (stroke (width 0.12) (type solid)) (layer "F.SilkS"))
  (pad "1" thru_hole rect (at 0 0 270) (size 1.7 1.7) (drill 1) (layers "*.Cu" "*.Mask") (remove_unused_layers no) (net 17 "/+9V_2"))
  (pad "2" thru_hole oval (at 0 2.54 270) (size 1.7 1.7) (drill 1) (layers "*.Cu" "*.Mask") (remove_unused_layers no) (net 14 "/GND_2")))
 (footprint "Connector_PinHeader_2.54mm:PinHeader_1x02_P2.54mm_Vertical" (layer "F.Cu") (at 104.14 61.595 90)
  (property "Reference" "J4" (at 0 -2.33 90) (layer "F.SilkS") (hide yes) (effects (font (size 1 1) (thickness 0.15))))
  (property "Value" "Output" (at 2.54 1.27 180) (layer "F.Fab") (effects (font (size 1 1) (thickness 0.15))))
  (fp_line (start -1.33 -1.33) (end 0 -1.33) (stroke (width 0.12) (type solid)) (layer "F.SilkS"))
  (fp_line (start -1.33 0) (end -1.33 -1.33) (stroke (width 0.12) (type solid)) (layer "F.SilkS"))
  (fp_line (start 1.33 1.27) (end 1.33 3.87) (stroke (width 0.12) (type solid)) (layer "F.SilkS"))
  (fp_line (start -1.33 1.27) (end 1.33 1.27) (stroke (width 0.12) (type solid)) (layer "F.SilkS"))
  (fp_line (start -1.33 1.27) (end -1.33 3.87) (stroke (width 0.12) (type solid)) (layer "F.SilkS"))
  (fp_line (start -1.33 3.87) (end 1.33 3.87) (stroke (width 0.12) (type solid)) (layer "F.SilkS"))
  (pad "1" thru_hole rect (at 0 0 90) (size 1.7 1.7) (drill 1) (layers "*.Cu" "*.Mask") (remove_unused_layers no) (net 16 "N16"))
  (pad "2" thru_hole oval (at 0 2.54 90) (size 1.7 1.7) (drill 1) (layers "*.Cu" "*.Mask") (remove_unused_layers no) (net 2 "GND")))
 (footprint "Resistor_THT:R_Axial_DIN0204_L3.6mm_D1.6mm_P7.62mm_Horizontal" (layer "F.Cu") (at 99.06 92.075 180)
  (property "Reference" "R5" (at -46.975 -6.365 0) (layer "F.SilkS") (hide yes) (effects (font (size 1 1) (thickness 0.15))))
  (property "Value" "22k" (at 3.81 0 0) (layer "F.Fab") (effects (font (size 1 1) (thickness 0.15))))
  (fp_line (start 6.68 0) (end 5.73 0) (stroke (width 0.12) (type solid)) (layer "F.SilkS"))
  (fp_line (start 5.73 0.92) (end 5.73 -0.92) (stroke (width 0.12) (type solid)) (layer "F.SilkS"))
  (fp_line (start 5.73 -0.92) (end 1.89 -0.92) (stroke (width 0.12) (type solid)) (layer "F.SilkS"))
  (fp_line (start 1.89 0.92) (end 5.73 0.92) (stroke (width 0.12) (type solid)) (layer "F.SilkS"))
  (fp_line (start 1.89 -0.92) (end 1.89 0.92) (stroke (width 0.12) (type solid)) (layer "F.SilkS"))
  (fp_line (start 0.94 0) (end 1.89 0) (stroke (width 0.12) (type solid)) (layer "F.SilkS"))
  (pad "1" thru_hole circle (at 0 0 180) (size 1.4 1.4) (drill 0.7) (layers "*.Cu" "*.Mask") (remove_unused_layers no) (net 5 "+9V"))
  (pad "2" thru_hole oval (at 7.62 0 180) (size 1.4 1.4) (drill 0.7) (layers "*.Cu" "*.Mask") (remove_unused_layers no) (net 11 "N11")))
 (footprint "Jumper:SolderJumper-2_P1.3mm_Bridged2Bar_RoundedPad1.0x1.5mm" (layer "B.Cu") (at 91.44 66.675 -90)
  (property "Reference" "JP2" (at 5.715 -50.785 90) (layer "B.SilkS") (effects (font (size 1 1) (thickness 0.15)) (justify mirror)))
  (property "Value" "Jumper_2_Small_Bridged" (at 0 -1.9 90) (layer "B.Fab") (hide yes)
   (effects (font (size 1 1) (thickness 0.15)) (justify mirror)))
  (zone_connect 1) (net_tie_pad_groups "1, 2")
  (fp_rect (start 0.254 0.508) (end 2.286 -0.508) (stroke (width 0.2) (type solid)) (fill solid) (layer "B.Cu"))
  (pad "1" smd custom (at 0 0 270) (size 1 0.5) (layers "B.Cu" "B.Mask") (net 17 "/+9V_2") (zone_connect 2) (thermal_bridge_angle 45)
   (options (clearance outline) (anchor rect)) (primitives))
  (pad "2" smd custom (at 2.54 0 270) (size 1 0.5) (layers "B.Cu" "B.Mask") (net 2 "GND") (zone_connect 2) (thermal_bridge_angle 45)
   (options (clearance outline) (anchor rect)) (primitives)))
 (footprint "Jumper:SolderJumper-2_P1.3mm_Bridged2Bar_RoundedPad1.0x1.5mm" (layer "B.Cu") (at 91.44 59.055 90)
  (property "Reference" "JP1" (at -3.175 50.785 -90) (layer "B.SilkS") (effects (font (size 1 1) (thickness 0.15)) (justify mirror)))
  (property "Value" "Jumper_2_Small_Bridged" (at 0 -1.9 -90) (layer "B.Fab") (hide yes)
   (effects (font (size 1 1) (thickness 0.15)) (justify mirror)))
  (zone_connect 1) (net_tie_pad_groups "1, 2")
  (fp_rect (start 0.254 0.508) (end 2.286 -0.508) (stroke (width 0.2) (type solid)) (fill solid) (layer "B.Cu"))
  (pad "1" smd custom (at 0 0 90) (size 1 0.5) (layers "B.Cu" "B.Mask") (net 9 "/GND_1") (zone_connect 2) (thermal_bridge_angle 45)
   (options (clearance outline) (anchor rect)) (primitives))
  (pad "2" smd custom (at 2.54 0 90) (size 1 0.5) (layers "B.Cu" "B.Mask") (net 2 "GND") (zone_connect 2) (thermal_bridge_angle 45)
   (options (clearance outline) (anchor rect)) (primitives)))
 (gr_rect (start 48.26 53.975) (end 111.76 102.235) (stroke (width 0.05) (type default)) (fill none) (layer "Edge.Cuts"))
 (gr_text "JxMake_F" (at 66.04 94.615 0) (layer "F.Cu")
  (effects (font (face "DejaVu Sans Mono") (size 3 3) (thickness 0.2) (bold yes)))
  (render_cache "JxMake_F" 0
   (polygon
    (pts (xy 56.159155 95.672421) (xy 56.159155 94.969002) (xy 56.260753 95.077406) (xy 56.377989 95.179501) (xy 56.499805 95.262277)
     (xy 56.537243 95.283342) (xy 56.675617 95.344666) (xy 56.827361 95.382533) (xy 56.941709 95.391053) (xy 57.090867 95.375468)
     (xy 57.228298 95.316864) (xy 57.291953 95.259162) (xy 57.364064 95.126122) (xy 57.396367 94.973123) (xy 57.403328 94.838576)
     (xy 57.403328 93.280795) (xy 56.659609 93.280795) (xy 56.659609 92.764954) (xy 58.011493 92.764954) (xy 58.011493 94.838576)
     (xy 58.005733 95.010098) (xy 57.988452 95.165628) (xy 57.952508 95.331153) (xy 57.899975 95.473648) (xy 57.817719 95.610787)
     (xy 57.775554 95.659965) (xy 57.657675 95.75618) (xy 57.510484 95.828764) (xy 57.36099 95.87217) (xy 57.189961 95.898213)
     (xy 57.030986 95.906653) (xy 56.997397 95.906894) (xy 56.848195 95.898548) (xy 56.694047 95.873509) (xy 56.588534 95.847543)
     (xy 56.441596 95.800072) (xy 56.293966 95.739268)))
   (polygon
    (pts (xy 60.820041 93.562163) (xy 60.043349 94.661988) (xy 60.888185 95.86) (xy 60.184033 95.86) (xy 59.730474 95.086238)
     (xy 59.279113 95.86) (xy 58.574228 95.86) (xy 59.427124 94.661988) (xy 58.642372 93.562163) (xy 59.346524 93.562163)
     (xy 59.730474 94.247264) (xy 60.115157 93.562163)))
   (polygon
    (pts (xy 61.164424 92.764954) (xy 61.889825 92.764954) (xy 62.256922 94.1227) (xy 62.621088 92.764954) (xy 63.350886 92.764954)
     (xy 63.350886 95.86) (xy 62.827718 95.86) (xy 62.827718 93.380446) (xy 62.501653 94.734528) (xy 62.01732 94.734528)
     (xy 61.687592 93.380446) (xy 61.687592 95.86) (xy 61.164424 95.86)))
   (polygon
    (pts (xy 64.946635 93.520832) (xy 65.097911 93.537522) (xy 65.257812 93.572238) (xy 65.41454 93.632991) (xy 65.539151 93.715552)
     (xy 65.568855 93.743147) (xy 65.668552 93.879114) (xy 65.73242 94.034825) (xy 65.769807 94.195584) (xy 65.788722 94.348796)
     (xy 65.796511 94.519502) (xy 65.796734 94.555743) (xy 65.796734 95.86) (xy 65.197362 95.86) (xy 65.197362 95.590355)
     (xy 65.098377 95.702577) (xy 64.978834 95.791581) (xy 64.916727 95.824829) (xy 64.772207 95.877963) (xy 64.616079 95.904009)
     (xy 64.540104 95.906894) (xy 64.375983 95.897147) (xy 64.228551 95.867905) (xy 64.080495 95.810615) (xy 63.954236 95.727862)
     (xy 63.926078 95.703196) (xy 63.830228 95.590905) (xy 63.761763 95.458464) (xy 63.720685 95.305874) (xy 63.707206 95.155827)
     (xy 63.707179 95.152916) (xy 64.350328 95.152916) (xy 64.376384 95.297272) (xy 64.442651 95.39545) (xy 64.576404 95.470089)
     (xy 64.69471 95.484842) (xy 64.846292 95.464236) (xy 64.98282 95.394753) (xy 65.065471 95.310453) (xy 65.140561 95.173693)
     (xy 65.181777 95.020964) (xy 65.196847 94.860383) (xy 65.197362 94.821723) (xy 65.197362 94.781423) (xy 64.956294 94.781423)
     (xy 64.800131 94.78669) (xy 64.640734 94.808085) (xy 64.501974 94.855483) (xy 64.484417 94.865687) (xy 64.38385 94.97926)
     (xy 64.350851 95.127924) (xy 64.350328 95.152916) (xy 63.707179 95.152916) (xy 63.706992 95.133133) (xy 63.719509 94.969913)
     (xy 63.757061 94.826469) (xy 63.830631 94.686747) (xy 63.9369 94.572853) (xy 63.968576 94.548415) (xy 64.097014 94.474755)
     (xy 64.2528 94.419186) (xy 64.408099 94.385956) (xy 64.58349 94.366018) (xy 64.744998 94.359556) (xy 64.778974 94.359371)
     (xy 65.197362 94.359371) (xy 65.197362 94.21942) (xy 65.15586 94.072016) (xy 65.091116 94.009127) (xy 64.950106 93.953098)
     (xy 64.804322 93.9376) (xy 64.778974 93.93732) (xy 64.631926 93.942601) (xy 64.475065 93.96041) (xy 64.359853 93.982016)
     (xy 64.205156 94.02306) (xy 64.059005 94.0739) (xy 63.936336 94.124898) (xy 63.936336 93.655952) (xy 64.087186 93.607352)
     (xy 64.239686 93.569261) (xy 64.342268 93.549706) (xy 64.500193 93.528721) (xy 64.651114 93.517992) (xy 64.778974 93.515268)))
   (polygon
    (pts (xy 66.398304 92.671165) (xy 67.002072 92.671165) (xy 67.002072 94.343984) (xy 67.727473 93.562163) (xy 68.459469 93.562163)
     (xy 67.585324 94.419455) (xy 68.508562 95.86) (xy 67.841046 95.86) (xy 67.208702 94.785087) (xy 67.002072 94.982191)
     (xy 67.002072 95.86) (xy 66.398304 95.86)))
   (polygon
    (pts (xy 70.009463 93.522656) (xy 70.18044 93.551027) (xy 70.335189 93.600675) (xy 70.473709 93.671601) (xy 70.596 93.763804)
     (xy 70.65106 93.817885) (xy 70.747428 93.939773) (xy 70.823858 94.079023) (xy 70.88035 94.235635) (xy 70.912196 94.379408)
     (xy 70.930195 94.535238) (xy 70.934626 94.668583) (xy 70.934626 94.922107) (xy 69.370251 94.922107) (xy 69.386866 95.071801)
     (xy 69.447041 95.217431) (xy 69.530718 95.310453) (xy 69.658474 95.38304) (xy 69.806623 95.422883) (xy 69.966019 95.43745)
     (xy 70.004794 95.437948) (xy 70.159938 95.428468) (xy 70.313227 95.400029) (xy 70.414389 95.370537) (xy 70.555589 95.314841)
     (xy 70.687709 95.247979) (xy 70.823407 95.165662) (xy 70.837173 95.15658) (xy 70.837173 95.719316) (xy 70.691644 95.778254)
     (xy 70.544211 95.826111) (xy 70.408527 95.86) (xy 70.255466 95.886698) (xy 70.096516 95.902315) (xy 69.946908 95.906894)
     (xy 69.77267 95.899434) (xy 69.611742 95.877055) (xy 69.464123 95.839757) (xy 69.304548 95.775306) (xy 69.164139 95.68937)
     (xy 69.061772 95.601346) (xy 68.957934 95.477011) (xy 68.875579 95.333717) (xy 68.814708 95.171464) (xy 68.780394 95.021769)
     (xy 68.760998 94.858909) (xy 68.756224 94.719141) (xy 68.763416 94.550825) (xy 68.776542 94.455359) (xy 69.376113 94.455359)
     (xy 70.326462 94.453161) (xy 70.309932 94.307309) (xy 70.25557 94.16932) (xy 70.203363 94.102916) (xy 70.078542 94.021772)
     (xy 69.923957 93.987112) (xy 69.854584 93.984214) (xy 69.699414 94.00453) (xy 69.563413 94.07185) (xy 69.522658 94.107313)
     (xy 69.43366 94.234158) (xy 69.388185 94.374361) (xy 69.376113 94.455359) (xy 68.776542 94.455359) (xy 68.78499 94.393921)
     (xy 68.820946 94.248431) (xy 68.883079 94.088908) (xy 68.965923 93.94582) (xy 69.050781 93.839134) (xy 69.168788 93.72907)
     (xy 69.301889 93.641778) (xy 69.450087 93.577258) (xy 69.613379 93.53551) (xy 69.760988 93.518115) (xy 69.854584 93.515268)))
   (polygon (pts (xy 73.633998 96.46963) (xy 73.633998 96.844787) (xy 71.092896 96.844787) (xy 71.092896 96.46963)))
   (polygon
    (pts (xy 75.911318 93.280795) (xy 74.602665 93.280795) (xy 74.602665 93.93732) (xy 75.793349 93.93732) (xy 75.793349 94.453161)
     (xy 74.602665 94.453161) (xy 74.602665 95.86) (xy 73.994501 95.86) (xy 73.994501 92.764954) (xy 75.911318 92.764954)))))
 (segment (start 104.14 99.695) (end 109.22 99.695) (width 1) (layer "B.Cu") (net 2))
 (segment (start 91.44 56.515) (end 109.22 56.515) (width 1) (layer "B.Cu") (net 2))
 (segment (start 96.44 86.995) (end 83.82 86.995) (width 1) (layer "B.Cu") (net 2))
 (segment (start 83.82 86.995) (end 83.82 97.155) (width 1) (layer "B.Cu") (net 2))
 (segment (start 106.68 89.535) (end 109.22 89.535) (width 1) (layer "B.Cu") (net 2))
 (segment (start 83.82 86.995) (end 83.82 69.215) (width 1) (layer "B.Cu") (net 2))
 (segment (start 91.44 97.155) (end 86.36 97.155) (width 1) (layer "B.Cu") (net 2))
 (segment (start 96.44 84.455) (end 96.44 86.995) (width 1) (layer "B.Cu") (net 2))
 (segment (start 91.44 56.515) (end 83.82 56.515) (width 1) (layer "B.Cu") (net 2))
 (segment (start 91.44 69.215) (end 83.82 69.215) (width 1) (layer "B.Cu") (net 2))
 (segment (start 109.22 99.695) (end 109.22 61.595) (width 1) (layer "B.Cu") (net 2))
 (segment (start 106.68 61.595) (end 109.22 61.595) (width 1) (layer "B.Cu") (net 2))
 (segment (start 83.82 97.155) (end 86.36 97.155) (width 1) (layer "B.Cu") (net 2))
 (segment (start 83.82 56.515) (end 83.82 69.215) (width 1) (layer "B.Cu") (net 2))
 (segment (start 109.22 56.515) (end 109.22 61.595) (width 1) (layer "B.Cu") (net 2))
 (segment (start 104.14 79.375) (end 104.14 84.455) (width 0.2) (layer "F.Cu") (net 5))
 (via (at 104.14 84.455) (size 1.6) (drill 1) (layers "F.Cu" "B.Cu") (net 5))
 (via (at 104.14 79.375) (size 1.6) (drill 1) (layers "F.Cu" "B.Cu") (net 5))
 (segment (start 99.06 92.075) (end 99.06 84.455) (width 1) (layer "B.Cu") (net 5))
 (segment (start 106.68 79.375) (end 104.14 79.375) (width 1) (layer "B.Cu") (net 5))
 (segment (start 99.06 61.515) (end 99.06 66.675) (width 1) (layer "B.Cu") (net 5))
 (segment (start 91.44 61.595) (end 96.52 61.595) (width 1) (layer "B.Cu") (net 5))
 (segment (start 99.06 84.455) (end 104.14 84.455) (width 1) (layer "B.Cu") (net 5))
 (segment (start 106.68 66.675) (end 106.68 79.375) (width 1) (layer "B.Cu") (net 5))
 (segment (start 96.52 61.595) (end 99.06 61.595) (width 1) (layer "B.Cu") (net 5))
 (segment (start 99.06 66.675) (end 106.68 66.675) (width 1) (layer "B.Cu") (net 5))
 (segment (start 93.98 64.135) (end 93.98 81.915) (width 1) (layer "B.Cu") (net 10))
 (segment (start 91.44 84.455) (end 91.44 81.915) (width 1) (layer "B.Cu") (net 10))
 (segment (start 91.44 64.135) (end 93.98 64.135) (width 1) (layer "B.Cu") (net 10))
 (segment (start 93.98 81.915) (end 91.44 81.915) (width 1) (layer "B.Cu") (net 10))
 (segment (start 86.36 84.455) (end 91.44 84.455) (width 1) (layer "B.Cu") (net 10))
 (segment (start 88.9 59.055) (end 88.9 61.555) (width 1) (layer "B.Cu") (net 8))
 (segment (start 88.9 66.675) (end 88.9 64.175) (width 1) (layer "B.Cu") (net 14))
 (segment (start 101.6 97.155) (end 101.6 99.695) (width 1) (layer "B.Cu") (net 3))
 (segment (start 101.6 89.535) (end 101.6 92.155) (width 1) (layer "B.Cu") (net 4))
 (segment (start 104.14 61.595) (end 104.14 64.215) (width 1) (layer "B.Cu") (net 16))
 (segment (start 99.06 71.755) (end 104.14 71.755) (width 1) (layer "B.Cu") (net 12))
 (segment (start 104.14 71.755) (end 104.14 69.215) (width 1) (layer "B.Cu") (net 12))
 (segment (start 99.06 81.915) (end 99.06 71.755) (width 1) (layer "B.Cu") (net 12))
 (segment (start 101.6 76.835) (end 101.6 81.915) (width 1) (layer "B.Cu") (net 7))
 (segment (start 106.68 81.915) (end 101.6 81.915) (width 1) (layer "B.Cu") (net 7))
 (segment (start 96.52 69.215) (end 96.52 76.835) (width 1) (layer "B.Cu") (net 6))
 (segment (start 91.44 92.075) (end 91.44 94.615) (width 1) (layer "B.Cu") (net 11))
 (segment (start 86.36 94.615) (end 86.36 92.075) (width 1) (layer "B.Cu") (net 1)))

